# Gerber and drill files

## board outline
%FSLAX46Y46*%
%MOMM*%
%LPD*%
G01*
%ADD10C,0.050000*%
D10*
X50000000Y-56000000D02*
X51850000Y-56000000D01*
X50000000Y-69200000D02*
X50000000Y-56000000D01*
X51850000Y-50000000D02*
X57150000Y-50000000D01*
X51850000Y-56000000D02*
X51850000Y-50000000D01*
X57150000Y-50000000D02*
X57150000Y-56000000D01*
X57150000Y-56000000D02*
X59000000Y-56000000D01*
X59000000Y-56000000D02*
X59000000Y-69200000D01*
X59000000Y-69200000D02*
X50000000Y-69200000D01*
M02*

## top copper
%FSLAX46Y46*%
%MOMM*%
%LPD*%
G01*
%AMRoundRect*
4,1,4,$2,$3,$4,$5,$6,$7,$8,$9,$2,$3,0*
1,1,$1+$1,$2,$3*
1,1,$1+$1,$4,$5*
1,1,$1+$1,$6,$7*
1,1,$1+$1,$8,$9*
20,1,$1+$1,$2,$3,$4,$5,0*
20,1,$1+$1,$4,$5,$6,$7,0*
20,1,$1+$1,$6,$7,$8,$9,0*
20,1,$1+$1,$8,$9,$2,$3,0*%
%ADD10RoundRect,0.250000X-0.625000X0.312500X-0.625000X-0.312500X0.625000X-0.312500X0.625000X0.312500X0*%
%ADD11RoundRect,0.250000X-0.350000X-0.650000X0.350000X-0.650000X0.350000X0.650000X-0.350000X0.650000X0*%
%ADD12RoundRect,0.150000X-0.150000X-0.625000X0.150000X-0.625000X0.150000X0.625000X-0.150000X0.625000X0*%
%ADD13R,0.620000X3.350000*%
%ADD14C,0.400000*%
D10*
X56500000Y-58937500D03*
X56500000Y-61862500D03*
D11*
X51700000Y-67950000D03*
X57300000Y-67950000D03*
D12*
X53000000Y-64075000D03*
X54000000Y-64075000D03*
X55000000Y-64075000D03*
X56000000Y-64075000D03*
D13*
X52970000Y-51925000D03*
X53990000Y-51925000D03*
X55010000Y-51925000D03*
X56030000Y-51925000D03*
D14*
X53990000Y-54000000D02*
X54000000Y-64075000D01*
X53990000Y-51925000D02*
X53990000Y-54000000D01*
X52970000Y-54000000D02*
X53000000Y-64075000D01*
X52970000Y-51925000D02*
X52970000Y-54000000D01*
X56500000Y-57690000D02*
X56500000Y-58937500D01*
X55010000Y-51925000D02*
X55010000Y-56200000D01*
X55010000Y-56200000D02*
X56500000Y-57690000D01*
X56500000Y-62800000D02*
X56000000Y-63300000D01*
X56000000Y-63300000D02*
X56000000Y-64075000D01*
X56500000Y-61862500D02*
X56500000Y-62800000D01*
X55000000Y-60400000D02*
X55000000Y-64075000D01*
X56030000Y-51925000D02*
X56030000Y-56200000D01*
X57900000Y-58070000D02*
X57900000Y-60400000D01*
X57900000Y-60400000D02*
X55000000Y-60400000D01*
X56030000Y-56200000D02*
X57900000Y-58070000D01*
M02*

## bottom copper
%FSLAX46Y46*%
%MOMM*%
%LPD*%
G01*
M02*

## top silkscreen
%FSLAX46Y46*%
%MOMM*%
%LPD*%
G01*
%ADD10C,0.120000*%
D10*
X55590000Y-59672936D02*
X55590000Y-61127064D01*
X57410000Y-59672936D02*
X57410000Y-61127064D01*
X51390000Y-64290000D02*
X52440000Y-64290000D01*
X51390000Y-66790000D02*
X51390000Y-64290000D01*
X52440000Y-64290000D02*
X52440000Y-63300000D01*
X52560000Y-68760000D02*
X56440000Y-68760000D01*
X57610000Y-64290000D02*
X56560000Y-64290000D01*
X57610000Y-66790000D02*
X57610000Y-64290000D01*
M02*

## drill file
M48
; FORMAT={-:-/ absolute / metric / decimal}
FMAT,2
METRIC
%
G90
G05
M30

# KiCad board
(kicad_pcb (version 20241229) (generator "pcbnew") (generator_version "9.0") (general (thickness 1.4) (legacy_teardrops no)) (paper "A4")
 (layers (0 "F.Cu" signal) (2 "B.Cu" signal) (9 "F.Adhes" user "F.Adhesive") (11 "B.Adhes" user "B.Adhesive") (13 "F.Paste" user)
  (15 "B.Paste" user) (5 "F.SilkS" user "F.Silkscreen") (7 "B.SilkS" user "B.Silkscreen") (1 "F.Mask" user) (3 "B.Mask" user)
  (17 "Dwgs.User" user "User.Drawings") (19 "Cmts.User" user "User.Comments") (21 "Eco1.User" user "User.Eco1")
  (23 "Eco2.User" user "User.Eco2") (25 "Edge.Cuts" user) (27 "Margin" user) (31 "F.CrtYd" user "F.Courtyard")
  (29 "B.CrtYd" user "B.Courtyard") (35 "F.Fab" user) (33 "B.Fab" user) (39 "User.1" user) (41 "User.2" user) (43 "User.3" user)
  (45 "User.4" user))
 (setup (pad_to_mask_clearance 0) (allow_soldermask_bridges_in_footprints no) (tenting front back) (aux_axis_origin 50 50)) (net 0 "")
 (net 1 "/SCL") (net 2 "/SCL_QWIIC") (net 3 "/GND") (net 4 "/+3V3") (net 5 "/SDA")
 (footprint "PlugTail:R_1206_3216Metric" (layer "F.Cu") (at 56.5 60.4 -90)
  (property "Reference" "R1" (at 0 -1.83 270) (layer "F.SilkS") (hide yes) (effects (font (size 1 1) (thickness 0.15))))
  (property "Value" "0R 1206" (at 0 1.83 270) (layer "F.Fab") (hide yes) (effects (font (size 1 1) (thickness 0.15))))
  (fp_line (start -0.727064 0.91) (end 0.727064 0.91) (stroke (width 0.12) (type solid)) (layer "F.SilkS"))
  (fp_line (start -0.727064 -0.91) (end 0.727064 -0.91) (stroke (width 0.12) (type solid)) (layer "F.SilkS"))
  (pad "1" smd roundrect (at -1.4625 0 270) (size 1.125 1.75) (layers "F.Cu" "F.Mask" "F.Paste") (roundrect_rratio 0.222222) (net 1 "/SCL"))
  (pad "2" smd roundrect (at 1.4625 0 270) (size 1.125 1.75) (layers "F.Cu" "F.Mask" "F.Paste") (roundrect_rratio 0.222222)
   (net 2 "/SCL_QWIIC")))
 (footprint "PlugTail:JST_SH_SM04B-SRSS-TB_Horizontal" (layer "F.Cu") (at 54.5 66.075)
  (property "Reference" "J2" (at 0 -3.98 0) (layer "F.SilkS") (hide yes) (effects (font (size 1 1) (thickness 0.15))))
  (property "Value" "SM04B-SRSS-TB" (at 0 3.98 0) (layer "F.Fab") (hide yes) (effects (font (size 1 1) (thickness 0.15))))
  (fp_line (start -3.11 -1.785) (end -2.06 -1.785) (stroke (width 0.12) (type solid)) (layer "F.SilkS"))
  (fp_line (start -3.11 0.715) (end -3.11 -1.785) (stroke (width 0.12) (type solid)) (layer "F.SilkS"))
  (fp_line (start -2.06 -1.785) (end -2.06 -2.775) (stroke (width 0.12) (type solid)) (layer "F.SilkS"))
  (fp_line (start -1.94 2.685) (end 1.94 2.685) (stroke (width 0.12) (type solid)) (layer "F.SilkS"))
  (fp_line (start 3.11 -1.785) (end 2.06 -1.785) (stroke (width 0.12) (type solid)) (layer "F.SilkS"))
  (fp_line (start 3.11 0.715) (end 3.11 -1.785) (stroke (width 0.12) (type solid)) (layer "F.SilkS"))
  (pad "" smd roundrect (at -2.8 1.875) (size 1.2 1.8) (layers "F.Cu" "F.Mask" "F.Paste") (roundrect_rratio 0.208333))
  (pad "" smd roundrect (at 2.8 1.875) (size 1.2 1.8) (layers "F.Cu" "F.Mask" "F.Paste") (roundrect_rratio 0.208333))
  (pad "1" smd roundrect (at -1.5 -2) (size 0.6 1.55) (layers "F.Cu" "F.Mask" "F.Paste") (roundrect_rratio 0.25) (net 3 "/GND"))
  (pad "2" smd roundrect (at -0.5 -2) (size 0.6 1.55) (layers "F.Cu" "F.Mask" "F.Paste") (roundrect_rratio 0.25) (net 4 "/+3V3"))
  (pad "3" smd roundrect (at 0.5 -2) (size 0.6 1.55) (layers "F.Cu" "F.Mask" "F.Paste") (roundrect_rratio 0.25) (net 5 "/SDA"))
  (pad "4" smd roundrect (at 1.5 -2) (size 0.6 1.55) (layers "F.Cu" "F.Mask" "F.Paste") (roundrect_rratio 0.25) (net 2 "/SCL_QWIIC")))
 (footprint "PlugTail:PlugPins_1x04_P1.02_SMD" (layer "F.Cu") (at 54.5 50)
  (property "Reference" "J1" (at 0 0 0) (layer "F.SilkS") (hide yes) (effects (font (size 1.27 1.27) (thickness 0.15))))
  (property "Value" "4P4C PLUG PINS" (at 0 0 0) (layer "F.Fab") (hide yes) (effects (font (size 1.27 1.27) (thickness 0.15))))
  (pad "1" smd rect (at -1.53 1.925) (size 0.62 3.35) (layers "F.Cu" "F.Mask") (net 3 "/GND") (thermal_bridge_angle 45))
  (pad "2" smd rect (at -0.51 1.925) (size 0.62 3.35) (layers "F.Cu" "F.Mask") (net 4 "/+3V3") (thermal_bridge_angle 45))
  (pad "3" smd rect (at 0.51 1.925) (size 0.62 3.35) (layers "F.Cu" "F.Mask") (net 1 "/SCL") (thermal_bridge_angle 45))
  (pad "4" smd rect (at 1.53 1.925) (size 0.62 3.35) (layers "F.Cu" "F.Mask") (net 5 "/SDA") (thermal_bridge_angle 45)))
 (gr_line (start 50 56) (end 51.85 56) (stroke (width 0.05) (type default)) (layer "Edge.Cuts"))
 (gr_line (start 50 69.2) (end 50 56) (stroke (width 0.05) (type default)) (layer "Edge.Cuts"))
 (gr_line (start 51.85 50) (end 57.15 50) (stroke (width 0.05) (type default)) (layer "Edge.Cuts"))
 (gr_line (start 51.85 56) (end 51.85 50) (stroke (width 0.05) (type default)) (layer "Edge.Cuts"))
 (gr_line (start 57.15 50) (end 57.15 56) (stroke (width 0.05) (type default)) (layer "Edge.Cuts"))
 (gr_line (start 57.15 56) (end 59 56) (stroke (width 0.05) (type default)) (layer "Edge.Cuts"))
 (gr_line (start 59 56) (end 59 69.2) (stroke (width 0.05) (type default)) (layer "Edge.Cuts"))
 (gr_line (start 59 69.2) (end 50 69.2) (stroke (width 0.05) (type default)) (layer "Edge.Cuts"))
 (segment (start 53.99 54) (end 54 64.075) (width 0.4) (layer "F.Cu") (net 4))
 (segment (start 53.99 51.925) (end 53.99 54) (width 0.4) (layer "F.Cu") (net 4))
 (segment (start 52.97 54) (end 53 64.075) (width 0.4) (layer "F.Cu") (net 3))
 (segment (start 52.97 51.925) (end 52.97 54) (width 0.4) (layer "F.Cu") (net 3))
 (segment (start 56.5 57.69) (end 56.5 58.9375) (width 0.4) (layer "F.Cu") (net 1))
 (segment (start 55.01 51.925) (end 55.01 56.2) (width 0.4) (layer "F.Cu") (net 1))
 (segment (start 55.01 56.2) (end 56.5 57.69) (width 0.4) (layer "F.Cu") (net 1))
 (segment (start 56.5 62.8) (end 56 63.3) (width 0.4) (layer "F.Cu") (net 2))
 (segment (start 56 63.3) (end 56 64.075) (width 0.4) (layer "F.Cu") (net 2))
 (segment (start 56.5 61.8625) (end 56.5 62.8) (width 0.4) (layer "F.Cu") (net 2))
 (segment (start 55 60.4) (end 55 64.075) (width 0.4) (layer "F.Cu") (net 5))
 (segment (start 56.03 51.925) (end 56.03 56.2) (width 0.4) (layer "F.Cu") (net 5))
 (segment (start 57.9 58.07) (end 57.9 60.4) (width 0.4) (layer "F.Cu") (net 5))
 (segment (start 57.9 60.4) (end 55 60.4) (width 0.4) (layer "F.Cu") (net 5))
 (segment (start 56.03 56.2) (end 57.9 58.07) (width 0.4) (layer "F.Cu") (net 5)))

